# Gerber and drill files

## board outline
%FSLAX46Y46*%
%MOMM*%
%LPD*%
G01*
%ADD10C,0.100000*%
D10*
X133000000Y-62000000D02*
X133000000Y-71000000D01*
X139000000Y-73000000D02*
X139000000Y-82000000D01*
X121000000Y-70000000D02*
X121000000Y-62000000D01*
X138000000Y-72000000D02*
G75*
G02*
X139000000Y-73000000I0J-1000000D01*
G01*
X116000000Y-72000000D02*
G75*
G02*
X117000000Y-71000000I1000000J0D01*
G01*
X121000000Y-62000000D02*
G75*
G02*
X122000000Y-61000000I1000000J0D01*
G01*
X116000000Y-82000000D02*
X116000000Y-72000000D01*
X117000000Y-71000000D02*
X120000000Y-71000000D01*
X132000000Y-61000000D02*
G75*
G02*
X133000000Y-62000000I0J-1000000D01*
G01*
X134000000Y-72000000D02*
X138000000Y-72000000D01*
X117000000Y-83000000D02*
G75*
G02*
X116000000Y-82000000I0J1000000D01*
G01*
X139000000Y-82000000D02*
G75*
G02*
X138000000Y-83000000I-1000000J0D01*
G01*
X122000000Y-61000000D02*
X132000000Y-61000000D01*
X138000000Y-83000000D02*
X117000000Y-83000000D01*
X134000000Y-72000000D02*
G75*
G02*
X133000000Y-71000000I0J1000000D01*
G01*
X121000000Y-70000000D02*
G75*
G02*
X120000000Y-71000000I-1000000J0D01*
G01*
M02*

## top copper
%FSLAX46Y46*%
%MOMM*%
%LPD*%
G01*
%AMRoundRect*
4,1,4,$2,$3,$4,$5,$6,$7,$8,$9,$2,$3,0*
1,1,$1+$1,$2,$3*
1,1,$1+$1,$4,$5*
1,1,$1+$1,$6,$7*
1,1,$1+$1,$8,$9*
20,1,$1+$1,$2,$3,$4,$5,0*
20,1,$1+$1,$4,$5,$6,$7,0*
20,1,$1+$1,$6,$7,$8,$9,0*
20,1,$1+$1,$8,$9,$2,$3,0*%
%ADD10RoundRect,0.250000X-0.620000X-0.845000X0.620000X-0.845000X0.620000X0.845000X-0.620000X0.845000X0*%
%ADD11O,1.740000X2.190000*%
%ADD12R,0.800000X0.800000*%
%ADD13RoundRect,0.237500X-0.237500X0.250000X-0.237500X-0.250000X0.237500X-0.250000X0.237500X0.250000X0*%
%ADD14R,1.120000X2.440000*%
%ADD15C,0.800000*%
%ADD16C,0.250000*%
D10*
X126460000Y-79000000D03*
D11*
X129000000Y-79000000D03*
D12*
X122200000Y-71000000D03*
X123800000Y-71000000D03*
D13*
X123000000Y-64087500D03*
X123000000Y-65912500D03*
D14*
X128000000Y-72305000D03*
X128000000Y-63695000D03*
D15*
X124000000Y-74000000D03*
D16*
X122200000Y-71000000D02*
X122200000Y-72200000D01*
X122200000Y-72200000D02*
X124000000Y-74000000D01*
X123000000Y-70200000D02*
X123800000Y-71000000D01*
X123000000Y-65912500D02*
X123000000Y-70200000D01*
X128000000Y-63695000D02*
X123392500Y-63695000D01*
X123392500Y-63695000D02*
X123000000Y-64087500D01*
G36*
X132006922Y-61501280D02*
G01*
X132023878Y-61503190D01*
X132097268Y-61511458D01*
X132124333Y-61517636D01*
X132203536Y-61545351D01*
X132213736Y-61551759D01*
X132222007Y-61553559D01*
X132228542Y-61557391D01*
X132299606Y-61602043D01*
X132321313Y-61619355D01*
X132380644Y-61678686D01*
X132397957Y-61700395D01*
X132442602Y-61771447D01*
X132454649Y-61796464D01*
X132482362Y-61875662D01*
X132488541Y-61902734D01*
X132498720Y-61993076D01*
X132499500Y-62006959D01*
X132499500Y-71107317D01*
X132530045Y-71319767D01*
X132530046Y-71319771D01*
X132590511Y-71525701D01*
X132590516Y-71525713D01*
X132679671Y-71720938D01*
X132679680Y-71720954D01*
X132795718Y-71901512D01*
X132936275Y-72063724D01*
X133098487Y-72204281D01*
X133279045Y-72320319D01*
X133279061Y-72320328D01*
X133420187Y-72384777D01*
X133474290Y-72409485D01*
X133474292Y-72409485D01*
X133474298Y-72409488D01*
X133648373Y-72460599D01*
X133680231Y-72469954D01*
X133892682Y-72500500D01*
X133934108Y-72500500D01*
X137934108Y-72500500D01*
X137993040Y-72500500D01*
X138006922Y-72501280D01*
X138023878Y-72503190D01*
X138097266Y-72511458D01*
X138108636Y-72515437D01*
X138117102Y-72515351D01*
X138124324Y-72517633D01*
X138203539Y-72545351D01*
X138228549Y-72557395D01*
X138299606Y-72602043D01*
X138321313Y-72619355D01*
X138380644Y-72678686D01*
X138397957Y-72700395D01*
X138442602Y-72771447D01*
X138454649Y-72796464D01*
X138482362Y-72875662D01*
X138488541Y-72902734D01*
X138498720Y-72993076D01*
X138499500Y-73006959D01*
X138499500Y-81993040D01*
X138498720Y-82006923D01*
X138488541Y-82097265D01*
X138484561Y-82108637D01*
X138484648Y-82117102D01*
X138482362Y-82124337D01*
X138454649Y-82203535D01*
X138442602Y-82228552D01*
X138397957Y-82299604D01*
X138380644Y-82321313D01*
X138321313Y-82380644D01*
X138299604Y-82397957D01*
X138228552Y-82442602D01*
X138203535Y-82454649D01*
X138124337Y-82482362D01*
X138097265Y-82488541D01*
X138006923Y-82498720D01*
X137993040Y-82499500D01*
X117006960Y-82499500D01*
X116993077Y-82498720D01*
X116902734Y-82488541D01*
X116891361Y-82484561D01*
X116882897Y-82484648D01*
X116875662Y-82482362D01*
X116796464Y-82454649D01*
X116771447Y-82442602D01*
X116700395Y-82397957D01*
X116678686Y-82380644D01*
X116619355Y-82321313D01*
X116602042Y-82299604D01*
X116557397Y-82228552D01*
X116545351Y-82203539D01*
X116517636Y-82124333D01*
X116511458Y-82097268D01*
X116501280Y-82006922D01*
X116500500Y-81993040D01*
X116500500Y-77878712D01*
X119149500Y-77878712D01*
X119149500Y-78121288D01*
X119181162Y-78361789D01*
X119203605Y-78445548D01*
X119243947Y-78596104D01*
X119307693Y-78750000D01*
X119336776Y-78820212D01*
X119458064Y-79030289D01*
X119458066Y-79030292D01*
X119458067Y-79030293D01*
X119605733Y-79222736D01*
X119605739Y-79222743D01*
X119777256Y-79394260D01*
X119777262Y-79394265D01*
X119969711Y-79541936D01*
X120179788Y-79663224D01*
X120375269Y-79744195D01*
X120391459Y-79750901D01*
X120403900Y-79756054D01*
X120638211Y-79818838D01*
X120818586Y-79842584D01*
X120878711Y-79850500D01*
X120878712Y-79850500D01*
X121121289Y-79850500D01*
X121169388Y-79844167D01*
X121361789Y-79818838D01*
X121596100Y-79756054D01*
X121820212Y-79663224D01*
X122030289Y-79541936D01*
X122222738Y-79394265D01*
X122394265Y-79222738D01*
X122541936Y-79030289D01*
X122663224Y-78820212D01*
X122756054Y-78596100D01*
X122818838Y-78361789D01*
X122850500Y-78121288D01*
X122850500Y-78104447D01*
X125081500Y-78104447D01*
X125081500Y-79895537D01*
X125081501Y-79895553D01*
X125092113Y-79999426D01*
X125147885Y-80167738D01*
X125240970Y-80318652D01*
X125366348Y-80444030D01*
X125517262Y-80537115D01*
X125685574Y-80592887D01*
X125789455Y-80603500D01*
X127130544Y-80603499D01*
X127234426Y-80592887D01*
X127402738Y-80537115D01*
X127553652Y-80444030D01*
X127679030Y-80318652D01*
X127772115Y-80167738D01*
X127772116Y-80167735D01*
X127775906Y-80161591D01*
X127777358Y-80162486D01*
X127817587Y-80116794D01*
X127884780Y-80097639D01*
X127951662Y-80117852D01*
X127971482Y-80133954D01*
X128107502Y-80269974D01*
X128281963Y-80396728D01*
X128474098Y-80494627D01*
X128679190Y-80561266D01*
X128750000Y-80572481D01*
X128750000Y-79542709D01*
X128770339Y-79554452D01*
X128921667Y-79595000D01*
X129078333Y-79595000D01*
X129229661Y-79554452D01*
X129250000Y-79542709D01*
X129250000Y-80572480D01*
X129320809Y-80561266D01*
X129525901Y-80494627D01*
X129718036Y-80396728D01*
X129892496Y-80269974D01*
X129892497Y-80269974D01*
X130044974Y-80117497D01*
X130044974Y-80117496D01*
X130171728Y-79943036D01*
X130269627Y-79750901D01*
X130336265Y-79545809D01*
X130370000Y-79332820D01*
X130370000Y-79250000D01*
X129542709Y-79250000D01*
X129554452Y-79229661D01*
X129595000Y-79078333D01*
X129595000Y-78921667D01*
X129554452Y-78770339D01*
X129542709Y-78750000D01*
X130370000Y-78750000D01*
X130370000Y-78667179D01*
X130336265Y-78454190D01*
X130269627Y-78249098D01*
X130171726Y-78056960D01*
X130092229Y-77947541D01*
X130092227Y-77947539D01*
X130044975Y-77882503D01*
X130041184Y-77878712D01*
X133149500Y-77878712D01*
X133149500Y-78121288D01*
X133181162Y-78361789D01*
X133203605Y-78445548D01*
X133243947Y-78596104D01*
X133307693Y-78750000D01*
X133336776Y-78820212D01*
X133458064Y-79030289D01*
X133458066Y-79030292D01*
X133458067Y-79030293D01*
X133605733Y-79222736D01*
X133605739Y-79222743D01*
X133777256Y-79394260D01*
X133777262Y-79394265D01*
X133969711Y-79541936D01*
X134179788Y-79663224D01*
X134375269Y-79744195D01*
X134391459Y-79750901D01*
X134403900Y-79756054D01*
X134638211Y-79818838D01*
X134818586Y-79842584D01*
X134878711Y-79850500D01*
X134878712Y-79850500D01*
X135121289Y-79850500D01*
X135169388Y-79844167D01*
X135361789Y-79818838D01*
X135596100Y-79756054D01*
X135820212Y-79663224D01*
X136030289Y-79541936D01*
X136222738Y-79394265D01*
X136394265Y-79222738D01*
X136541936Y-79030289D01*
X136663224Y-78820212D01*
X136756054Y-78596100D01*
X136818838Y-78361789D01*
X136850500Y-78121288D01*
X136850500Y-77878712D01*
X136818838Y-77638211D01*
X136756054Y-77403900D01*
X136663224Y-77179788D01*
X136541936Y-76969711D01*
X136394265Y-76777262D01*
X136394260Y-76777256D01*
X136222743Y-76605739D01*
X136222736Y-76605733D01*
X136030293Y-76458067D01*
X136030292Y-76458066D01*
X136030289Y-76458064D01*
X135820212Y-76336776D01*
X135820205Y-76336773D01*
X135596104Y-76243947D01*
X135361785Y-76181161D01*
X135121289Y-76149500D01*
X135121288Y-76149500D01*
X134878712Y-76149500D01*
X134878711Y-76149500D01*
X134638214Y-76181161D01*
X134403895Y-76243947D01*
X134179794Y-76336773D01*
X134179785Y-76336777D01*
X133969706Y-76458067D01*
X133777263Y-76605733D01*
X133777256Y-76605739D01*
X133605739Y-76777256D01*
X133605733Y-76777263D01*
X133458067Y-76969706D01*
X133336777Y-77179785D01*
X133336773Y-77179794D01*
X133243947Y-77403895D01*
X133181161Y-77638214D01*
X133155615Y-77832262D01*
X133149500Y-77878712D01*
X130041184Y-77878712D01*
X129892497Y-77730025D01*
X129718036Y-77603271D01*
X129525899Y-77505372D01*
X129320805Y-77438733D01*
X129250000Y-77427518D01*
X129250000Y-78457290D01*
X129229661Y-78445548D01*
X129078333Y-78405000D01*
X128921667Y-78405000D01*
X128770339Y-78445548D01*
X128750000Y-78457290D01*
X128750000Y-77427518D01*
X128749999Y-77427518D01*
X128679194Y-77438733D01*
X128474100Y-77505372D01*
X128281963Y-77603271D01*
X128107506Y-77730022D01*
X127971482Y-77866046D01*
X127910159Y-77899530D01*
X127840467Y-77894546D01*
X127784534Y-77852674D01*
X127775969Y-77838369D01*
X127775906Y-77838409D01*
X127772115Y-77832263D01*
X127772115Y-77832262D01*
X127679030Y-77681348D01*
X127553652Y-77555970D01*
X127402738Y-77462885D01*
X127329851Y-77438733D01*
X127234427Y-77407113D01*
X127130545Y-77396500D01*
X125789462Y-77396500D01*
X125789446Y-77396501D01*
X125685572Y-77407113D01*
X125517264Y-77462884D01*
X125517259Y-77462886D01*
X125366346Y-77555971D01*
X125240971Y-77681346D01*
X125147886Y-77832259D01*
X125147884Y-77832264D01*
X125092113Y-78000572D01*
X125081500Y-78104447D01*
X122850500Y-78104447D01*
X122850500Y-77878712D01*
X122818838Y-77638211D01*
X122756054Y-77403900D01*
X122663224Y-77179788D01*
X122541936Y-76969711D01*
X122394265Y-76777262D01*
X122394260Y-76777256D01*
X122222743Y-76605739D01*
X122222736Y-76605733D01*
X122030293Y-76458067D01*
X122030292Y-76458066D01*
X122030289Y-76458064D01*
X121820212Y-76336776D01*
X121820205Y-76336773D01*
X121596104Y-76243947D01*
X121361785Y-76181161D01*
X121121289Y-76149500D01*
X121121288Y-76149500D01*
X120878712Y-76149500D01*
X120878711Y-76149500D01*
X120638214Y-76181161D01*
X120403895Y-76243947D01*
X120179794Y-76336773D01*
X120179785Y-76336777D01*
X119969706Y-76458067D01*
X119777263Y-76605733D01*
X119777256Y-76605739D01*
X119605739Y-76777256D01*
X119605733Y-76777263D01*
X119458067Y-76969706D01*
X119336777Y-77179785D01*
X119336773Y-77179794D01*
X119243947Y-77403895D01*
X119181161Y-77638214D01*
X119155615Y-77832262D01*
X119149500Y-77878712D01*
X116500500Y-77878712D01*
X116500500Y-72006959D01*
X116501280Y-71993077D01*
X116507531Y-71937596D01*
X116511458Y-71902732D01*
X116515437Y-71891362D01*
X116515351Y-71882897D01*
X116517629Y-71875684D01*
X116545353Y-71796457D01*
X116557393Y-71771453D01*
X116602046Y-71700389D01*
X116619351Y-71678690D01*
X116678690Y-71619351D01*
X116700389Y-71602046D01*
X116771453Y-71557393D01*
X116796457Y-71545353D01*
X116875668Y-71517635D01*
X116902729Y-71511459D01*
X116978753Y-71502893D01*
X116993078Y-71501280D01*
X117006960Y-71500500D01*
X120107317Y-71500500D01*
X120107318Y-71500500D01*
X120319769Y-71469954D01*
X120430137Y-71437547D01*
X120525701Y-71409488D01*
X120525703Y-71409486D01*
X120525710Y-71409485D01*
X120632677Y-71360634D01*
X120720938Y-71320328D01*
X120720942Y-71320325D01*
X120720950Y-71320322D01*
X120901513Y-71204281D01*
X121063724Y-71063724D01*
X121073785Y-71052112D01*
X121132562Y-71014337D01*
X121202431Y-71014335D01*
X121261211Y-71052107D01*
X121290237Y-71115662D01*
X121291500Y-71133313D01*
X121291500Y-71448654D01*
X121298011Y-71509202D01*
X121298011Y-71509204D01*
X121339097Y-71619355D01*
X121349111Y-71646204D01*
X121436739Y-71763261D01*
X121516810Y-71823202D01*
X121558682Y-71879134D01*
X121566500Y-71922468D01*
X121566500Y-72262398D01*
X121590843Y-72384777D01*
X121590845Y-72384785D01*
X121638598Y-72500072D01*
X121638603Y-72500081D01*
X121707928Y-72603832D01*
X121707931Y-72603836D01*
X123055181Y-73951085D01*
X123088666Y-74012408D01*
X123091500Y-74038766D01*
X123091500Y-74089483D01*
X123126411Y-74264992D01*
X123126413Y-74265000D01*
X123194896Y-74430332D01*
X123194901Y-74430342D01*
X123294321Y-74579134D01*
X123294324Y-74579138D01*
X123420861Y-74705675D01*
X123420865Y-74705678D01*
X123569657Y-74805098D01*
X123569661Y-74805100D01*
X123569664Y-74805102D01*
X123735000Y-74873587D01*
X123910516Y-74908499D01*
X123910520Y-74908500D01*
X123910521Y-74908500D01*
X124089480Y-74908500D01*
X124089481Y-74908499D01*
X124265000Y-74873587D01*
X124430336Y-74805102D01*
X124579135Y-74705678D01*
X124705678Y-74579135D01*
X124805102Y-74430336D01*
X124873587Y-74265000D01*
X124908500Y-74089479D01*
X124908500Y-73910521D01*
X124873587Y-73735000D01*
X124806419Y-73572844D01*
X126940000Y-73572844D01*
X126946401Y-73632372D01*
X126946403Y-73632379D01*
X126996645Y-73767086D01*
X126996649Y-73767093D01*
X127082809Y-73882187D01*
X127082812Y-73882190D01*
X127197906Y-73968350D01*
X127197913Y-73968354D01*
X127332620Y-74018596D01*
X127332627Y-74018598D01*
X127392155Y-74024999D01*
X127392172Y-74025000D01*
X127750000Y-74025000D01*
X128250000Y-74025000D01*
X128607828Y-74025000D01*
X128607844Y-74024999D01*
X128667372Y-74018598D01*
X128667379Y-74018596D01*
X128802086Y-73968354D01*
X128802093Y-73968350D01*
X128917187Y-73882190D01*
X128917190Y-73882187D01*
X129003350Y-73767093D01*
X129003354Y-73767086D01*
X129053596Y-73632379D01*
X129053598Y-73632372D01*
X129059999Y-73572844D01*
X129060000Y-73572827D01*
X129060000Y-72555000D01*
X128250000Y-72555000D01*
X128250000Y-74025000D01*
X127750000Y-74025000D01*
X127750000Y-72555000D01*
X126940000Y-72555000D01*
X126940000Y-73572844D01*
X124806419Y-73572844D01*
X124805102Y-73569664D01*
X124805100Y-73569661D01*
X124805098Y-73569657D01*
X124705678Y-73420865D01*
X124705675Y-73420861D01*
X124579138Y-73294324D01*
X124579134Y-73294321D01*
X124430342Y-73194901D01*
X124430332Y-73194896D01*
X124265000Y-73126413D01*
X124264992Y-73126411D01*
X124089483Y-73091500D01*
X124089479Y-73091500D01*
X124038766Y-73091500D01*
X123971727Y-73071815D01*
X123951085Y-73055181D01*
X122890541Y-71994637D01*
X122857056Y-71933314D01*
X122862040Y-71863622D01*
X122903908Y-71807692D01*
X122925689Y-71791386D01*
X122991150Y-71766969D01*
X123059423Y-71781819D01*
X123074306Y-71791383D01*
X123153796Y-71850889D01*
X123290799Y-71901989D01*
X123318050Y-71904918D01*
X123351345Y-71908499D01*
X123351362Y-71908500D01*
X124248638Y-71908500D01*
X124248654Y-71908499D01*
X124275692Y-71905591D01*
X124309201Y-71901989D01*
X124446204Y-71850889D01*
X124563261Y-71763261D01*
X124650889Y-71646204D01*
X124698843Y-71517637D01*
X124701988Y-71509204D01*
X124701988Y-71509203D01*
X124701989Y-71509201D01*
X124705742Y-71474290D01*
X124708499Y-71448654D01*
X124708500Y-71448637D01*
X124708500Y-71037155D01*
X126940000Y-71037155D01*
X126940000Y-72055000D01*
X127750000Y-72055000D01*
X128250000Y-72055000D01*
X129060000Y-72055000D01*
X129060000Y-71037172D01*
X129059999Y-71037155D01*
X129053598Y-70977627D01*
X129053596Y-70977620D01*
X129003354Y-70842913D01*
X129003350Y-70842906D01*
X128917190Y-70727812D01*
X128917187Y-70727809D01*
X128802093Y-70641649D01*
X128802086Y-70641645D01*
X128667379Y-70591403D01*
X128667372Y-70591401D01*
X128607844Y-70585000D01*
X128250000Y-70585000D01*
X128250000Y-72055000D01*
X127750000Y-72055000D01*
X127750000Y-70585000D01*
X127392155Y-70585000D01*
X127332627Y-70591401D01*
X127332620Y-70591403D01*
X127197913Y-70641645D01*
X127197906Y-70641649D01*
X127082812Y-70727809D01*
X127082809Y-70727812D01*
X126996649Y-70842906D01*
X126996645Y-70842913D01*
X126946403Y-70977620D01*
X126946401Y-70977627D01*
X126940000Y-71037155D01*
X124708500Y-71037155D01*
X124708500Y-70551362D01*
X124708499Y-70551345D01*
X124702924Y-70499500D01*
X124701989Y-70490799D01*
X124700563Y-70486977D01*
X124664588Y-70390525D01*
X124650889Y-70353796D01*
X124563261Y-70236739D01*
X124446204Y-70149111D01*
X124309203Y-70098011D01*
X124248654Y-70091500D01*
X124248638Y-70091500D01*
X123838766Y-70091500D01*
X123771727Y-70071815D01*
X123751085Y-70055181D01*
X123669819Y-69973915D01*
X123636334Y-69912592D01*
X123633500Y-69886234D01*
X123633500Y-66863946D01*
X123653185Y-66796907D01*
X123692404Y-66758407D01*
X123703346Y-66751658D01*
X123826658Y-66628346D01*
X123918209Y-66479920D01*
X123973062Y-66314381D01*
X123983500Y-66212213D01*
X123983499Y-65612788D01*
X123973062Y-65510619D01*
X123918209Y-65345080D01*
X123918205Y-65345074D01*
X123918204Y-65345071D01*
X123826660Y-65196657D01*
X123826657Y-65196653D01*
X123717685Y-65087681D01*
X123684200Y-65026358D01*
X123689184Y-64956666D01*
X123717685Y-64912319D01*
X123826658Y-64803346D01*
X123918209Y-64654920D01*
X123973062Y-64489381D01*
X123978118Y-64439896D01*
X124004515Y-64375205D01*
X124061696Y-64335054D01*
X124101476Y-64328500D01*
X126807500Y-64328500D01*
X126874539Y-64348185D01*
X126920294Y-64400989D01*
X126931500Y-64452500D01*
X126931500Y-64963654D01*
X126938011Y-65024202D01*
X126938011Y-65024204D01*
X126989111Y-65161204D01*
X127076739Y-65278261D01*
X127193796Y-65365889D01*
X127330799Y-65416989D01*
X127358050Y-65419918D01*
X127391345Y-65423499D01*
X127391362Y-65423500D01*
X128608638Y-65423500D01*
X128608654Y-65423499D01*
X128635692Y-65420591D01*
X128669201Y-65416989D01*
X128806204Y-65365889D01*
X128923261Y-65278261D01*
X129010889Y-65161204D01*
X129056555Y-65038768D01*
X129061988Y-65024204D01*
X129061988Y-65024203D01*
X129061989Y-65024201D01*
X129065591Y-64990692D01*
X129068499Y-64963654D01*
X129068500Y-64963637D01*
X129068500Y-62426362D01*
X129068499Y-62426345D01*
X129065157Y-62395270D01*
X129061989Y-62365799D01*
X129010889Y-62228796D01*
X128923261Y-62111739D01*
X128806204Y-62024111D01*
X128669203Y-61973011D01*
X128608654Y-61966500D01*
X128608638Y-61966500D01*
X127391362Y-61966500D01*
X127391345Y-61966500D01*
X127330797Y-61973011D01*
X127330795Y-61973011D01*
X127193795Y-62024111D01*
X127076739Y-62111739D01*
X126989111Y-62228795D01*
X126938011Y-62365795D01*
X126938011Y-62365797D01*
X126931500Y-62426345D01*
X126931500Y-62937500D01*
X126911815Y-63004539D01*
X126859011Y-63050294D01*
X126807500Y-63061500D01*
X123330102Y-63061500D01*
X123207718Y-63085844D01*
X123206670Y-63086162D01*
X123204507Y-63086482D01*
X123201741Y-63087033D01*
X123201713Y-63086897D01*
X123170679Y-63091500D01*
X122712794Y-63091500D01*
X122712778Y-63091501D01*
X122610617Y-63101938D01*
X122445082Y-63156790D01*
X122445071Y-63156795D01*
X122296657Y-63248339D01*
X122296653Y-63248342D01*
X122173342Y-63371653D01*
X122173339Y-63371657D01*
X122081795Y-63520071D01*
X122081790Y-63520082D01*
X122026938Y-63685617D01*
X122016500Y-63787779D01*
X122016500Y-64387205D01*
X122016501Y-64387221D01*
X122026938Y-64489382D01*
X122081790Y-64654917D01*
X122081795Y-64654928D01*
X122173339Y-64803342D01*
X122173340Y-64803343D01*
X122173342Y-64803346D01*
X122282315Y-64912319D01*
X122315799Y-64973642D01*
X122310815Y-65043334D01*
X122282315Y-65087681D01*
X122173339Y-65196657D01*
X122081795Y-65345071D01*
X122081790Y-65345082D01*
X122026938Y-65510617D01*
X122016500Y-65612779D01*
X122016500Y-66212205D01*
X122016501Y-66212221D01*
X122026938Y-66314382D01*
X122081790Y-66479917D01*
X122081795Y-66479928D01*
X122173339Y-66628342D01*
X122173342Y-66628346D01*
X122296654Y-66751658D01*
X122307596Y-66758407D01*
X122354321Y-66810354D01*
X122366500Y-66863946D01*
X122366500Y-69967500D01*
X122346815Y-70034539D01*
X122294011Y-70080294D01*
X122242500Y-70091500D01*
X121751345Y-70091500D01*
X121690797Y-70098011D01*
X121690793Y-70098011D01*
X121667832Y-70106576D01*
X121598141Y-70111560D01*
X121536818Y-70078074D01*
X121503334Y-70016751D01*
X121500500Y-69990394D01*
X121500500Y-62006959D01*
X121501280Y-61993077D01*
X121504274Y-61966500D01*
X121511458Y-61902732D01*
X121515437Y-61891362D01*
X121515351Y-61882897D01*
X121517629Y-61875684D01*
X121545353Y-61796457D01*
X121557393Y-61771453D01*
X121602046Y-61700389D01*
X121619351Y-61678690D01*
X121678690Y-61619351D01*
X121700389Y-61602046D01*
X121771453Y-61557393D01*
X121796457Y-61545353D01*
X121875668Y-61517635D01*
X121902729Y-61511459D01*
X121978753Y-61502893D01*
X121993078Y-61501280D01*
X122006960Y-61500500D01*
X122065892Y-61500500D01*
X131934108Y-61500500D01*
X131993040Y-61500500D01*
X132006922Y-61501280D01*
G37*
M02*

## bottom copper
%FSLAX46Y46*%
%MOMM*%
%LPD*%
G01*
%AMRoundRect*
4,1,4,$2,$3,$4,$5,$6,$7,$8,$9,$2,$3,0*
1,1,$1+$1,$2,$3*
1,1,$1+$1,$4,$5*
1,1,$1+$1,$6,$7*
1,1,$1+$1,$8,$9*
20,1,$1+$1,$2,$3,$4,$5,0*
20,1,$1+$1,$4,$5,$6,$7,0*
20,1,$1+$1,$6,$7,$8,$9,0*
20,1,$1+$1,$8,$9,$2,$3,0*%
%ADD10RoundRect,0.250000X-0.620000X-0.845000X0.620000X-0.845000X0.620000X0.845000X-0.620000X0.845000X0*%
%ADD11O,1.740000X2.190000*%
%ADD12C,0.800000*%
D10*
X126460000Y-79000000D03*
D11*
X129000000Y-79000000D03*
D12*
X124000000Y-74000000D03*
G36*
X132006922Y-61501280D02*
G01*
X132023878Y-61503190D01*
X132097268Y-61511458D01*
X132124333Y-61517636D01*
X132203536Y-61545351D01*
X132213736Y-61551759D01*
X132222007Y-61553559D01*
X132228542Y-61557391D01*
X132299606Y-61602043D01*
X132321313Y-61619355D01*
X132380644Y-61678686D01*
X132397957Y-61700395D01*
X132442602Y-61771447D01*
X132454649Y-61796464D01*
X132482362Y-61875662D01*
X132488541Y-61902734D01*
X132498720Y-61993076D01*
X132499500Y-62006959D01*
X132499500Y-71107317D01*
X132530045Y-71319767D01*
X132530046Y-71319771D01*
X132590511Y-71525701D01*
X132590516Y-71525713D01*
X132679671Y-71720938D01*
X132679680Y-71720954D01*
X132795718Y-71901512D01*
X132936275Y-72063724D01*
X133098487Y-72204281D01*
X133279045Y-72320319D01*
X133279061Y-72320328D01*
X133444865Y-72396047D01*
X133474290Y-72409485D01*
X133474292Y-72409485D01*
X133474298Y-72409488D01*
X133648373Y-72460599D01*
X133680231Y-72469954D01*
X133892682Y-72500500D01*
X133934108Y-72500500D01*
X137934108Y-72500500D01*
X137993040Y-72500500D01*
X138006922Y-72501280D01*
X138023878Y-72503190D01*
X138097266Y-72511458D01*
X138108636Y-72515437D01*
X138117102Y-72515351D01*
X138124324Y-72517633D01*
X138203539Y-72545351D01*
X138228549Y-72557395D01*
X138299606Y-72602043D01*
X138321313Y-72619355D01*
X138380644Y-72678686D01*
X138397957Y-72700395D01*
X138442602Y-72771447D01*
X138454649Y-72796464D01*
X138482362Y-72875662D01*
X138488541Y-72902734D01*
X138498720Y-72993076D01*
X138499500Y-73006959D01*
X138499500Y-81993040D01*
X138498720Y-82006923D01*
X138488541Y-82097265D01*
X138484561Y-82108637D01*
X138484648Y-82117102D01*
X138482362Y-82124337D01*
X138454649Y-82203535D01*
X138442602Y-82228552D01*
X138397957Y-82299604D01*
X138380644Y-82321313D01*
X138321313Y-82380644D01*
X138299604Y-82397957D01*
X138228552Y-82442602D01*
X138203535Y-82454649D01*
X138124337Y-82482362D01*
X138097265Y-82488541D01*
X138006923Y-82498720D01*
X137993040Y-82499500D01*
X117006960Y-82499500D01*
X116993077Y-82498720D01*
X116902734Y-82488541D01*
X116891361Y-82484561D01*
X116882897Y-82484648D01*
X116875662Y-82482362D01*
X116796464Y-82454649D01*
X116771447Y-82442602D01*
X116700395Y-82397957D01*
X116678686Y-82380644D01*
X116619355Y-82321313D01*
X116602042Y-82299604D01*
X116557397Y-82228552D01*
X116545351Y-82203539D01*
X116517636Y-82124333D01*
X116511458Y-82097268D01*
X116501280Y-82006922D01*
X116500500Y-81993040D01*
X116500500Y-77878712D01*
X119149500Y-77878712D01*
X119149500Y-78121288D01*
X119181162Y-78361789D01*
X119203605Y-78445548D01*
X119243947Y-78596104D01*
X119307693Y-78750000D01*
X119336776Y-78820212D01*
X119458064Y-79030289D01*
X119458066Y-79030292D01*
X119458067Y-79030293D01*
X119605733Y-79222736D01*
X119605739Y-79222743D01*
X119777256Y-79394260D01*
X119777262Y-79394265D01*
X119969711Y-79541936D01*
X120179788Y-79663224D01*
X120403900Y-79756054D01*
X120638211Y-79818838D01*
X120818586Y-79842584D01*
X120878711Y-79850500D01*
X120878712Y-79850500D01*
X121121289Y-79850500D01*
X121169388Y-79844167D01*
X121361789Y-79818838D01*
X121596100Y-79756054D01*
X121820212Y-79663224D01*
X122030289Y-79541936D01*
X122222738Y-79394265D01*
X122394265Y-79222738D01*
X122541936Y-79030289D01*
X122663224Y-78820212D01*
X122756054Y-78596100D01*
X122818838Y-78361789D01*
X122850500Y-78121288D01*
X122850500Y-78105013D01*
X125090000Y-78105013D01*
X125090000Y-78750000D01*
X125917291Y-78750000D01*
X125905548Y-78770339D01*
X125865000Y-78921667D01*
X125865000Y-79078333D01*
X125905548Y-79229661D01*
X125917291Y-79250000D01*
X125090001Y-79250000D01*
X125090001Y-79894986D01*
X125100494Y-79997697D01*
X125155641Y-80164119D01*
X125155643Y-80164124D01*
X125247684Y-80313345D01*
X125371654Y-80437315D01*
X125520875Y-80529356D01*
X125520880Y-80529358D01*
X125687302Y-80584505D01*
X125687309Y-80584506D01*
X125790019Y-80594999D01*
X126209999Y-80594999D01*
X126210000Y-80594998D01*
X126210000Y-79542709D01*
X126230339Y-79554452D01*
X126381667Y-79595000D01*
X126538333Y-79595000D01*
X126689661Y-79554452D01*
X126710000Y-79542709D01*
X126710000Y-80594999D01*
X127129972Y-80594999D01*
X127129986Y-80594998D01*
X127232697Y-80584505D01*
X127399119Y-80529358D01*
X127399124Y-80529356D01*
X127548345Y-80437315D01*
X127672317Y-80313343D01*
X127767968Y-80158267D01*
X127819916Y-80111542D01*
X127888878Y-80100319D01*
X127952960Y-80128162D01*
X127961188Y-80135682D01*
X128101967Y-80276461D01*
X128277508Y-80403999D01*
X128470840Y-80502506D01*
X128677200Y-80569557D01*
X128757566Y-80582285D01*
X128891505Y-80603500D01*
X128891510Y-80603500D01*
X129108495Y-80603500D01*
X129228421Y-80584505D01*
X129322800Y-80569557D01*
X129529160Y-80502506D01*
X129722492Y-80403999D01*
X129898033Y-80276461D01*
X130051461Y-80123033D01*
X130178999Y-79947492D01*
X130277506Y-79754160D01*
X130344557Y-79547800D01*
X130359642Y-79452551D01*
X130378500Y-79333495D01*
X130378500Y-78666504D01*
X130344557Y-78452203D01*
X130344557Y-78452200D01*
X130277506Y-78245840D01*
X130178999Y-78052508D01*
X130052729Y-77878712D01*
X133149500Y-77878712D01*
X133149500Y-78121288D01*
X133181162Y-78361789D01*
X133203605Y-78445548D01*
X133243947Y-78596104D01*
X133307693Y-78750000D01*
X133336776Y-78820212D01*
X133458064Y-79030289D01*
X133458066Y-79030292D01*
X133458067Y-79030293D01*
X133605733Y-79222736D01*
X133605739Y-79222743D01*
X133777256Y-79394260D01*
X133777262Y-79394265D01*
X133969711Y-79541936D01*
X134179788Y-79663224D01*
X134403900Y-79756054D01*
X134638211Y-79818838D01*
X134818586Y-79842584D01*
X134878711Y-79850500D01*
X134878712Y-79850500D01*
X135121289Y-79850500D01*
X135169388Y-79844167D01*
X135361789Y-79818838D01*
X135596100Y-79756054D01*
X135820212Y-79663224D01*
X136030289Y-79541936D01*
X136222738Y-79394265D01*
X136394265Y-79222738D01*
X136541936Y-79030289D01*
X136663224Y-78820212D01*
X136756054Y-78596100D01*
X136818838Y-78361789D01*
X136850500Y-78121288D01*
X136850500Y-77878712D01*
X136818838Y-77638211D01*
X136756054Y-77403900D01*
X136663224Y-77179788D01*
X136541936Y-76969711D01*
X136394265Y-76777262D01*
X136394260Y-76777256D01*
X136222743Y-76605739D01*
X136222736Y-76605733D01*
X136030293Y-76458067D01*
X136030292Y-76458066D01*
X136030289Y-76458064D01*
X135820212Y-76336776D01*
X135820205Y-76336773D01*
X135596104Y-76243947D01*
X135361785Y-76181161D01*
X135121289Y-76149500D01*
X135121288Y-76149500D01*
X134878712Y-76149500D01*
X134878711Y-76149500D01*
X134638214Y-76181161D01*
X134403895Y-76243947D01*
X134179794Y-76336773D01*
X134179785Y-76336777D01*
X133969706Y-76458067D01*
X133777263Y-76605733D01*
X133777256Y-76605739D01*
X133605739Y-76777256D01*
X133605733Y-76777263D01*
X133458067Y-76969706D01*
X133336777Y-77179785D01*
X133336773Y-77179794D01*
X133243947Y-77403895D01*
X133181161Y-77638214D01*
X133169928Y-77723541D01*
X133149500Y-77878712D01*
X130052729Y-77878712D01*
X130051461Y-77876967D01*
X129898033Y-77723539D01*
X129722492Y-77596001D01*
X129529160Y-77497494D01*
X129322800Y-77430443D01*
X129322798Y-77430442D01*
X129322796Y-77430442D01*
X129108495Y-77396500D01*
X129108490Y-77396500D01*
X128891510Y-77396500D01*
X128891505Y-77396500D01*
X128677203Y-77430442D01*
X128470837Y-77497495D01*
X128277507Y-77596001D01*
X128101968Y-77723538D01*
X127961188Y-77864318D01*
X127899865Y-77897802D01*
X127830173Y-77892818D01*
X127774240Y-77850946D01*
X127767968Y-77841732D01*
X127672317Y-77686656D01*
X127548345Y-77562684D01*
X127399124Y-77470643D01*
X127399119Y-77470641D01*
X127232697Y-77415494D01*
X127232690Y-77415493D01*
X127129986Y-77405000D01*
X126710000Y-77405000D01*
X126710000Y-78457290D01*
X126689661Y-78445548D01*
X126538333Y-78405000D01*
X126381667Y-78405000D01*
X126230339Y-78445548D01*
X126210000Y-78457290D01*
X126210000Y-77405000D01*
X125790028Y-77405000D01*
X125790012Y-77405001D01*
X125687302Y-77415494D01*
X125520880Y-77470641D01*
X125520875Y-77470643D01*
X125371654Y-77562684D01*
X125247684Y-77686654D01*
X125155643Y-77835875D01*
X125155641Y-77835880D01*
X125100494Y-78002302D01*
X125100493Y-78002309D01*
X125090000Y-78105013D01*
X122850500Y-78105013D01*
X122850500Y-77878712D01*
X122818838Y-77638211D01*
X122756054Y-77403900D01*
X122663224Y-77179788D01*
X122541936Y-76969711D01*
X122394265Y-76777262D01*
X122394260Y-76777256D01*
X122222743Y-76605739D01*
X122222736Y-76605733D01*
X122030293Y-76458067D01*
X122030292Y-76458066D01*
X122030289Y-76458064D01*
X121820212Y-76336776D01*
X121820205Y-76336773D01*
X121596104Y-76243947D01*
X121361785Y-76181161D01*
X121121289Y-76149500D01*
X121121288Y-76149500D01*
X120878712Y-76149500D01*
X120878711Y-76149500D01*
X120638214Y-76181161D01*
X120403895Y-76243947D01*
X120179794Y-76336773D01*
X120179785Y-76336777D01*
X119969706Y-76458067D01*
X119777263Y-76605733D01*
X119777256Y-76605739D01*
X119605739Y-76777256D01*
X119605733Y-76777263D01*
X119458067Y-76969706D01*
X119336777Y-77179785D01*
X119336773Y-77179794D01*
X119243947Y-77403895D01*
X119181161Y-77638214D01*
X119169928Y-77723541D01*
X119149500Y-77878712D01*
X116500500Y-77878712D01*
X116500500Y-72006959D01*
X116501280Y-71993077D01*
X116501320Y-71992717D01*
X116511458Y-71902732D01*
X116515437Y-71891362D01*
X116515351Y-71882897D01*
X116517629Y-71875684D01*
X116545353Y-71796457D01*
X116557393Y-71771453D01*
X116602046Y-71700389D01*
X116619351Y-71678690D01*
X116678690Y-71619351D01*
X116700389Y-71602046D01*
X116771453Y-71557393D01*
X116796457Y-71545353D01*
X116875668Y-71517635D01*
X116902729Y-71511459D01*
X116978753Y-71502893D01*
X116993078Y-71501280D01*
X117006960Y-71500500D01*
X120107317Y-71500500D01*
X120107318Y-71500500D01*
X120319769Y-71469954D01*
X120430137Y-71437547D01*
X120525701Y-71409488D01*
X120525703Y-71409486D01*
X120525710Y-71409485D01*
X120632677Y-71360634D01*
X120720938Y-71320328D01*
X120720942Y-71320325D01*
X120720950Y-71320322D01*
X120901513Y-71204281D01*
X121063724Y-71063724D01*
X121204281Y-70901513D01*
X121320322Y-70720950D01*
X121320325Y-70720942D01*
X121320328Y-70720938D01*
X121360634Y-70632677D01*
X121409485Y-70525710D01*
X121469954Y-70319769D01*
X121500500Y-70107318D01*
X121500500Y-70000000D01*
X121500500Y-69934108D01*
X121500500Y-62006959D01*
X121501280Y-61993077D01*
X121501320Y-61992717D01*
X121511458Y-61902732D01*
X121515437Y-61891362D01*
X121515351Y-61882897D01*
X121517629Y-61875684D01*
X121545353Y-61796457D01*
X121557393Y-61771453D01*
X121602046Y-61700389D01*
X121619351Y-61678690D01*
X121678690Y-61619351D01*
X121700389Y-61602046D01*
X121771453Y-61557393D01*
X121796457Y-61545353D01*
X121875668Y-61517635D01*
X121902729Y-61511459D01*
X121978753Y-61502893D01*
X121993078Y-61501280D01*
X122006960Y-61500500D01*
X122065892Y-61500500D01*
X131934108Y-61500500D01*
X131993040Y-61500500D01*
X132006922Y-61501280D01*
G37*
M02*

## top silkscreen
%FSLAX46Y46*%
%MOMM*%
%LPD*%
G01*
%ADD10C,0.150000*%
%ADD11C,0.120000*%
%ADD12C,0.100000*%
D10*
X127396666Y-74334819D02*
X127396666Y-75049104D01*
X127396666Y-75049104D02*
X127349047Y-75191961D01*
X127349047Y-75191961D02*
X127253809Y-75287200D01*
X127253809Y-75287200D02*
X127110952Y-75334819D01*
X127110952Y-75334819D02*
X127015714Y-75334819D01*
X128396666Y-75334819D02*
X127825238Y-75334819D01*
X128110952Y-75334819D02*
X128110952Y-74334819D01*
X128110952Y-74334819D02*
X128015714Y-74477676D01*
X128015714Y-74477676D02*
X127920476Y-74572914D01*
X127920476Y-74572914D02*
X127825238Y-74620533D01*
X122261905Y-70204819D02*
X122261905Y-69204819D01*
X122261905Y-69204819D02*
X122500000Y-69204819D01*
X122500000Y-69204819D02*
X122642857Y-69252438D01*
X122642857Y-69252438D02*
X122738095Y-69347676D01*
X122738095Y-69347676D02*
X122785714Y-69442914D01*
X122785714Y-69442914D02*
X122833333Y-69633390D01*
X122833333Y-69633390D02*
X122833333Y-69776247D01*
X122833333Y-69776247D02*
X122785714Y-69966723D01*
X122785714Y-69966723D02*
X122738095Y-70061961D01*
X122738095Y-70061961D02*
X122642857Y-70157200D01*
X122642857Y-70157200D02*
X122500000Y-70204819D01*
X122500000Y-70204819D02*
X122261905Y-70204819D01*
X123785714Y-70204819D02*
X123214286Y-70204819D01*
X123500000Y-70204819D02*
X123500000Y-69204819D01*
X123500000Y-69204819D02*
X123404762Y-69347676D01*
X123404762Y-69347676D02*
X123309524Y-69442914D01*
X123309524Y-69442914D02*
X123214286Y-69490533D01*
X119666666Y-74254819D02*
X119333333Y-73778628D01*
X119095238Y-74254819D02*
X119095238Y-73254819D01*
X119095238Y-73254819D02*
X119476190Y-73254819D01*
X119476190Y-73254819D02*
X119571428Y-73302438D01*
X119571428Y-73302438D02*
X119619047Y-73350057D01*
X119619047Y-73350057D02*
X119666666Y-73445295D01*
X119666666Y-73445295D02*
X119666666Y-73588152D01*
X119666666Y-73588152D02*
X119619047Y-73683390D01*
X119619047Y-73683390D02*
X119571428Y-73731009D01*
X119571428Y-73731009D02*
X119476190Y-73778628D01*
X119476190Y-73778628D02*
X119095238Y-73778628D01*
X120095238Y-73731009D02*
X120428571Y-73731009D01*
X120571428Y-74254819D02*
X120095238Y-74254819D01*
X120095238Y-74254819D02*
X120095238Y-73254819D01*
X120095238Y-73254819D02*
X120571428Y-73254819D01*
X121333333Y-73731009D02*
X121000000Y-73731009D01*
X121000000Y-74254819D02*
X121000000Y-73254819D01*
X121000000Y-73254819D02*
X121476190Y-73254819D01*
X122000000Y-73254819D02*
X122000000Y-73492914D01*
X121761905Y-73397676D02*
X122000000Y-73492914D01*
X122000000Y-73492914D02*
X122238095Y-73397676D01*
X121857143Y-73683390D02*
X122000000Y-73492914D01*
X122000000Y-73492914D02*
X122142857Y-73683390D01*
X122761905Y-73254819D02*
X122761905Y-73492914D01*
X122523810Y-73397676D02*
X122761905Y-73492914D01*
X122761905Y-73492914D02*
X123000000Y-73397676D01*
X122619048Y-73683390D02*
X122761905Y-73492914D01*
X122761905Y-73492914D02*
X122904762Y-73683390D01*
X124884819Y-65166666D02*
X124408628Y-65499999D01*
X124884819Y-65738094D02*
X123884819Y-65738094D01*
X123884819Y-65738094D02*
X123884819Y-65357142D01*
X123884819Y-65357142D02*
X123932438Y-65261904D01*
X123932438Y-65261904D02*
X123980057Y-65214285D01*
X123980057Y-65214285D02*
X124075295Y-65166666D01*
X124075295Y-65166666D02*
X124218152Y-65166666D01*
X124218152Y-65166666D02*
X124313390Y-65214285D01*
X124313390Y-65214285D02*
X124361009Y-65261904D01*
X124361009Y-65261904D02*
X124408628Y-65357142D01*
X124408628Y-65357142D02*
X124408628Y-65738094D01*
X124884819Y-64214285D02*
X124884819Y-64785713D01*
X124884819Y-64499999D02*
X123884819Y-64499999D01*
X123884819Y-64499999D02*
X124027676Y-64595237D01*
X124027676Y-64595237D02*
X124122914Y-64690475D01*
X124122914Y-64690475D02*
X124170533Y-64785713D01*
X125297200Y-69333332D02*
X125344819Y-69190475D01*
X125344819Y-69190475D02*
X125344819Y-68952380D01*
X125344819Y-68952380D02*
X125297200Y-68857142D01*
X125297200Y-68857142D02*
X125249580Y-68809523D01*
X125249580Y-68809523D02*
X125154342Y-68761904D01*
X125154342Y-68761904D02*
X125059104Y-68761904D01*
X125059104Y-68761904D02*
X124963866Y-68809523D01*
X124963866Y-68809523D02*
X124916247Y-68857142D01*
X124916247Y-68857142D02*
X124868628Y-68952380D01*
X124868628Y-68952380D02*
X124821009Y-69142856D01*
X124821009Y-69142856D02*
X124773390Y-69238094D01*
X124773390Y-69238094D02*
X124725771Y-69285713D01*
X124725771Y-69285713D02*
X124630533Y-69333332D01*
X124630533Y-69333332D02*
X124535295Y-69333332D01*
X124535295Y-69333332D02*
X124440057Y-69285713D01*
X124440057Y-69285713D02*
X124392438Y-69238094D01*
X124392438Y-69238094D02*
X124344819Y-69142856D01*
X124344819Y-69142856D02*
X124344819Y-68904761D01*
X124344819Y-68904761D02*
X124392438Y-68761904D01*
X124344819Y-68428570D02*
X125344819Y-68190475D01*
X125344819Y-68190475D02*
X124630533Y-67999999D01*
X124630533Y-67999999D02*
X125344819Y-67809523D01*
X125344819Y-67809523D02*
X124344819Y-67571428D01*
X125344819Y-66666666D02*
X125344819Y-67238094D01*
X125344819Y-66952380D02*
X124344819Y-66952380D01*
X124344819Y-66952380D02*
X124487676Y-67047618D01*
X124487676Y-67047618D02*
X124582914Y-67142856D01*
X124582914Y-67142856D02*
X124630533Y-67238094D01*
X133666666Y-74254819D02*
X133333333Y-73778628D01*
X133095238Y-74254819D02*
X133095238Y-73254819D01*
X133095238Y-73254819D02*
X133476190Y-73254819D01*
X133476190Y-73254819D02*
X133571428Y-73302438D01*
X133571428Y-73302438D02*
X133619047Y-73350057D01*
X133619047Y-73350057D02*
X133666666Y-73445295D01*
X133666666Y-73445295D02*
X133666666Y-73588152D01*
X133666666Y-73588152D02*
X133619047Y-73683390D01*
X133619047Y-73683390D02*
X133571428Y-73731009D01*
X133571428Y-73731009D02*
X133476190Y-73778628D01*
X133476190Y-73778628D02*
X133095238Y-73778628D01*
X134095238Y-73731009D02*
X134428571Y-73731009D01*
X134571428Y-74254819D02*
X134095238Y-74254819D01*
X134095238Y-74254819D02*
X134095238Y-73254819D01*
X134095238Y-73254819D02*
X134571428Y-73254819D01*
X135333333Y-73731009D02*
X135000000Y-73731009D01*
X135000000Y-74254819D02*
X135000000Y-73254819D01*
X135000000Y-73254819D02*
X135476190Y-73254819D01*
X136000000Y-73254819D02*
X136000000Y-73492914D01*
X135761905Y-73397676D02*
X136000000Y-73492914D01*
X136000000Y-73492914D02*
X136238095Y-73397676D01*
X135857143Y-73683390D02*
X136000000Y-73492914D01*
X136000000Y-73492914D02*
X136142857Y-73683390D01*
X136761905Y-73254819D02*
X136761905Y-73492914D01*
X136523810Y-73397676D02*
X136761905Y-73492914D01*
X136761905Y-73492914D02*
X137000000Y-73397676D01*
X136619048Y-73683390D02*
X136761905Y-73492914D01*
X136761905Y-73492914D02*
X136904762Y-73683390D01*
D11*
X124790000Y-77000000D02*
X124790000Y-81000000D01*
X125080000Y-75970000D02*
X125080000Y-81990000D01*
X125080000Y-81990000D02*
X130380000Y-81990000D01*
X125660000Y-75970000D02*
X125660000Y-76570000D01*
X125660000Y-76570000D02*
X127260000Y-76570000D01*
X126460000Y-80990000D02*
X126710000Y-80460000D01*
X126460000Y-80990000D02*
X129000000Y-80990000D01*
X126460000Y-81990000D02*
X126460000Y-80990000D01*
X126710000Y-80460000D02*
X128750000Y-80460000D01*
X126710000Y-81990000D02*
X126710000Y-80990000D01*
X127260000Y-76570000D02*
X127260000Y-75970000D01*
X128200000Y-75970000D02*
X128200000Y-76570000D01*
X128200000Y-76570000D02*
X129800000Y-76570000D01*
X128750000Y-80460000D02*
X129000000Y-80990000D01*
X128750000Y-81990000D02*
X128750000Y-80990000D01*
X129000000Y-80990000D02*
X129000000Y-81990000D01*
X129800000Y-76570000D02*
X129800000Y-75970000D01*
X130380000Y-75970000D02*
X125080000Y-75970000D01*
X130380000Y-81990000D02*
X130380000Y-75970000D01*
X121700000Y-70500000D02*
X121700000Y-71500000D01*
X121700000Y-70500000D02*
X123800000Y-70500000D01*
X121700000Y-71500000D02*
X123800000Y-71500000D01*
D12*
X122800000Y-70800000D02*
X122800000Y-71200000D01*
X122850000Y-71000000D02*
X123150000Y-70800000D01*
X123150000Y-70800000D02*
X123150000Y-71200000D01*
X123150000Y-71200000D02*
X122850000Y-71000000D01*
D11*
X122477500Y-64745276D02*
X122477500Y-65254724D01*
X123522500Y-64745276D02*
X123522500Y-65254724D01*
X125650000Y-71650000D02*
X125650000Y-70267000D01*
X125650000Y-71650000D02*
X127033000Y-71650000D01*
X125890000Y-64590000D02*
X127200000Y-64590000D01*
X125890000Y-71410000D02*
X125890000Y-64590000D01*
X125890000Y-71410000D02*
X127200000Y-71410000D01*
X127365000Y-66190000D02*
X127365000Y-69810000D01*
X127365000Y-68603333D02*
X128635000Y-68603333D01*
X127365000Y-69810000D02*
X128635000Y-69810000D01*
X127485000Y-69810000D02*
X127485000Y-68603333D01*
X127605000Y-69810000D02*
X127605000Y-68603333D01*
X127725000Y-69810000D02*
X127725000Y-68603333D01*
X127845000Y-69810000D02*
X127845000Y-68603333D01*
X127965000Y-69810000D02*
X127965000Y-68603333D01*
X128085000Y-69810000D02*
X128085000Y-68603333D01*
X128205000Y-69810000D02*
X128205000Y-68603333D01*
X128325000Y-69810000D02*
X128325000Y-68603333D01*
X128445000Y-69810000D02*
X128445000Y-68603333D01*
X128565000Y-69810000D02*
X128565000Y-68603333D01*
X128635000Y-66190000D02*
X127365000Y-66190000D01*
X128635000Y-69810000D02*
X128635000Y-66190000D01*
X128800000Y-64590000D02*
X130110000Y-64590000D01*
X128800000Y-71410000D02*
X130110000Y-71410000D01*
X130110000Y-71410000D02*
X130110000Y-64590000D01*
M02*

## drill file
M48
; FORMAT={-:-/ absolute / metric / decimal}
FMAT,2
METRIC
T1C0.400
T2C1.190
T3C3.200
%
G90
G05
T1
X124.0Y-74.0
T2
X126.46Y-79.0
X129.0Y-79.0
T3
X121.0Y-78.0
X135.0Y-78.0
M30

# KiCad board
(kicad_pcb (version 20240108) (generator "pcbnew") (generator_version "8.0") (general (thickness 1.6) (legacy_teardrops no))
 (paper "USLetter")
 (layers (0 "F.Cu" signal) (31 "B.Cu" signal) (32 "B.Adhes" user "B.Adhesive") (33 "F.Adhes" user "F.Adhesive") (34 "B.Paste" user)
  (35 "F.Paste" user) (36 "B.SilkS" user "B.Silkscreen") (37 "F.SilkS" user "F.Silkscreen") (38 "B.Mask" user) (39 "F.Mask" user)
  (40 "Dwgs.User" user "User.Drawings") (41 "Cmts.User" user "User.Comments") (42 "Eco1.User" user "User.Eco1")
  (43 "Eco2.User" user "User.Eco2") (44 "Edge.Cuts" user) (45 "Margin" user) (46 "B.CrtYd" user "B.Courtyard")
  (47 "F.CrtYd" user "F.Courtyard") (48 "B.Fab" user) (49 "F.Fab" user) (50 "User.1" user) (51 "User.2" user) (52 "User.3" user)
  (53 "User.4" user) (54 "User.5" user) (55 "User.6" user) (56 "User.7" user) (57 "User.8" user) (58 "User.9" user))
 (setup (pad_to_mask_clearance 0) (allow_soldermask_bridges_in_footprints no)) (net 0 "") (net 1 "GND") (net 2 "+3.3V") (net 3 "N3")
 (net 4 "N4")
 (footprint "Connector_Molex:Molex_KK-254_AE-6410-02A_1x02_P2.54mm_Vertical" (layer "F.Cu") (at 126.46 79)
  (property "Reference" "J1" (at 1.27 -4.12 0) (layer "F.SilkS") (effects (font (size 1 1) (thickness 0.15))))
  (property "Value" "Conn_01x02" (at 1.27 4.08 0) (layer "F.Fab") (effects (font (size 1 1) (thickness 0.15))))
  (fp_line (start -1.67 -2) (end -1.67 2) (stroke (width 0.12) (type solid)) (layer "F.SilkS"))
  (fp_line (start -1.38 -3.03) (end -1.38 2.99) (stroke (width 0.12) (type solid)) (layer "F.SilkS"))
  (fp_line (start -1.38 2.99) (end 3.92 2.99) (stroke (width 0.12) (type solid)) (layer "F.SilkS"))
  (fp_line (start -0.8 -3.03) (end -0.8 -2.43) (stroke (width 0.12) (type solid)) (layer "F.SilkS"))
  (fp_line (start -0.8 -2.43) (end 0.8 -2.43) (stroke (width 0.12) (type solid)) (layer "F.SilkS"))
  (fp_line (start 0 1.99) (end 0.25 1.46) (stroke (width 0.12) (type solid)) (layer "F.SilkS"))
  (fp_line (start 0 1.99) (end 2.54 1.99) (stroke (width 0.12) (type solid)) (layer "F.SilkS"))
  (fp_line (start 0 2.99) (end 0 1.99) (stroke (width 0.12) (type solid)) (layer "F.SilkS"))
  (fp_line (start 0.25 1.46) (end 2.29 1.46) (stroke (width 0.12) (type solid)) (layer "F.SilkS"))
  (fp_line (start 0.25 2.99) (end 0.25 1.99) (stroke (width 0.12) (type solid)) (layer "F.SilkS"))
  (fp_line (start 0.8 -2.43) (end 0.8 -3.03) (stroke (width 0.12) (type solid)) (layer "F.SilkS"))
  (fp_line (start 1.74 -3.03) (end 1.74 -2.43) (stroke (width 0.12) (type solid)) (layer "F.SilkS"))
  (fp_line (start 1.74 -2.43) (end 3.34 -2.43) (stroke (width 0.12) (type solid)) (layer "F.SilkS"))
  (fp_line (start 2.29 1.46) (end 2.54 1.99) (stroke (width 0.12) (type solid)) (layer "F.SilkS"))
  (fp_line (start 2.29 2.99) (end 2.29 1.99) (stroke (width 0.12) (type solid)) (layer "F.SilkS"))
  (fp_line (start 2.54 1.99) (end 2.54 2.99) (stroke (width 0.12) (type solid)) (layer "F.SilkS"))
  (fp_line (start 3.34 -2.43) (end 3.34 -3.03) (stroke (width 0.12) (type solid)) (layer "F.SilkS"))
  (fp_line (start 3.92 -3.03) (end -1.38 -3.03) (stroke (width 0.12) (type solid)) (layer "F.SilkS"))
  (fp_line (start 3.92 2.99) (end 3.92 -3.03) (stroke (width 0.12) (type solid)) (layer "F.SilkS"))
  (pad "1" thru_hole roundrect (at 0 0) (size 1.74 2.19) (drill 1.19) (layers "*.Cu" "*.Mask") (remove_unused_layers no)
   (roundrect_rratio 0.143678) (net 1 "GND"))
  (pad "2" thru_hole oval (at 2.54 0) (size 1.74 2.19) (drill 1.19) (layers "*.Cu" "*.Mask") (remove_unused_layers no) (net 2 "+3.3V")))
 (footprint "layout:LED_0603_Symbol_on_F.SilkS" (layer "F.Cu") (at 123 71)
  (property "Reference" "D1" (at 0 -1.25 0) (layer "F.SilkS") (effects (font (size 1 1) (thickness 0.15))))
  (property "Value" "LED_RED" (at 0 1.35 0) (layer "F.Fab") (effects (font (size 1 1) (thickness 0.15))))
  (fp_line (start -1.3 -0.5) (end -1.3 0.5) (stroke (width 0.12) (type solid)) (layer "F.SilkS"))
  (fp_line (start -1.3 -0.5) (end 0.8 -0.5) (stroke (width 0.12) (type solid)) (layer "F.SilkS"))
  (fp_line (start -1.3 0.5) (end 0.8 0.5) (stroke (width 0.12) (type solid)) (layer "F.SilkS"))
  (fp_line (start -0.2 -0.2) (end -0.2 0.2) (stroke (width 0.1) (type solid)) (layer "F.SilkS"))
  (fp_line (start -0.15 0) (end 0.15 -0.2) (stroke (width 0.1) (type solid)) (layer "F.SilkS"))
  (fp_line (start 0.15 -0.2) (end 0.15 0.2) (stroke (width 0.1) (type solid)) (layer "F.SilkS"))
  (fp_line (start 0.15 0.2) (end -0.15 0) (stroke (width 0.1) (type solid)) (layer "F.SilkS"))
  (pad "1" smd rect (at -0.8 0 180) (size 0.8 0.8) (layers "F.Cu" "F.Paste" "F.Mask") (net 1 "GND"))
  (pad "2" smd rect (at 0.8 0 180) (size 0.8 0.8) (layers "F.Cu" "F.Paste" "F.Mask") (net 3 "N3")))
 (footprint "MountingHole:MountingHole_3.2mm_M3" (layer "F.Cu") (at 121 78)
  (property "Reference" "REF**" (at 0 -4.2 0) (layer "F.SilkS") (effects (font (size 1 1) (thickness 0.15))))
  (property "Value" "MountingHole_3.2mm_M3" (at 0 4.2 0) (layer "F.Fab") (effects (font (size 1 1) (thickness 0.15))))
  (pad "" np_thru_hole circle (at 0 0) (size 3.2 3.2) (drill 3.2) (layers "*.Cu" "*.Mask")))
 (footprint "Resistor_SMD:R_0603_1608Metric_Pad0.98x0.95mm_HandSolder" (layer "F.Cu") (at 123 65 -90)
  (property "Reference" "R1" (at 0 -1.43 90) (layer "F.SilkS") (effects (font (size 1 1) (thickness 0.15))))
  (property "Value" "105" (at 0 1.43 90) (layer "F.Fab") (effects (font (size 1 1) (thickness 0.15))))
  (fp_line (start -0.254724 0.5225) (end 0.254724 0.5225) (stroke (width 0.12) (type solid)) (layer "F.SilkS"))
  (fp_line (start -0.254724 -0.5225) (end 0.254724 -0.5225) (stroke (width 0.12) (type solid)) (layer "F.SilkS"))
  (pad "1" smd roundrect (at -0.9125 0 270) (size 0.975 0.95) (layers "F.Cu" "F.Paste" "F.Mask") (roundrect_rratio 0.25) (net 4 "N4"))
  (pad "2" smd roundrect (at 0.9125 0 270) (size 0.975 0.95) (layers "F.Cu" "F.Paste" "F.Mask") (roundrect_rratio 0.25) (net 3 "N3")))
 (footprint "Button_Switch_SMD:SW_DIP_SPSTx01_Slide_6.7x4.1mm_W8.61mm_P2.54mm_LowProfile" (layer "F.Cu") (at 128 68 90)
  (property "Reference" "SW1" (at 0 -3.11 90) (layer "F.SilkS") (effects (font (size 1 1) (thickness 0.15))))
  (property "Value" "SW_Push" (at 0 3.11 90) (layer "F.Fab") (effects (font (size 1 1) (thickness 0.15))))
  (fp_line (start -3.65 -2.35) (end -2.267 -2.35) (stroke (width 0.12) (type solid)) (layer "F.SilkS"))
  (fp_line (start -3.65 -2.35) (end -3.65 -0.967) (stroke (width 0.12) (type solid)) (layer "F.SilkS"))
  (fp_line (start 3.41 -2.11) (end 3.41 -0.8) (stroke (width 0.12) (type solid)) (layer "F.SilkS"))
  (fp_line (start -3.41 -2.11) (end 3.41 -2.11) (stroke (width 0.12) (type solid)) (layer "F.SilkS"))
  (fp_line (start -3.41 -2.11) (end -3.41 -0.8) (stroke (width 0.12) (type solid)) (layer "F.SilkS"))
  (fp_line (start 1.81 -0.635) (end -1.81 -0.635) (stroke (width 0.12) (type solid)) (layer "F.SilkS"))
  (fp_line (start -0.603333 -0.635) (end -0.603333 0.635) (stroke (width 0.12) (type solid)) (layer "F.SilkS"))
  (fp_line (start -1.81 -0.635) (end -1.81 0.635) (stroke (width 0.12) (type solid)) (layer "F.SilkS"))
  (fp_line (start -1.81 -0.515) (end -0.603333 -0.515) (stroke (width 0.12) (type solid)) (layer "F.SilkS"))
  (fp_line (start -1.81 -0.395) (end -0.603333 -0.395) (stroke (width 0.12) (type solid)) (layer "F.SilkS"))
  (fp_line (start -1.81 -0.275) (end -0.603333 -0.275) (stroke (width 0.12) (type solid)) (layer "F.SilkS"))
  (fp_line (start -1.81 -0.155) (end -0.603333 -0.155) (stroke (width 0.12) (type solid)) (layer "F.SilkS"))
  (fp_line (start -1.81 -0.035) (end -0.603333 -0.035) (stroke (width 0.12) (type solid)) (layer "F.SilkS"))
  (fp_line (start -1.81 0.085) (end -0.603333 0.085) (stroke (width 0.12) (type solid)) (layer "F.SilkS"))
  (fp_line (start -1.81 0.205) (end -0.603333 0.205) (stroke (width 0.12) (type solid)) (layer "F.SilkS"))
  (fp_line (start -1.81 0.325) (end -0.603333 0.325) (stroke (width 0.12) (type solid)) (layer "F.SilkS"))
  (fp_line (start -1.81 0.445) (end -0.603333 0.445) (stroke (width 0.12) (type solid)) (layer "F.SilkS"))
  (fp_line (start -1.81 0.565) (end -0.603333 0.565) (stroke (width 0.12) (type solid)) (layer "F.SilkS"))
  (fp_line (start 1.81 0.635) (end 1.81 -0.635) (stroke (width 0.12) (type solid)) (layer "F.SilkS"))
  (fp_line (start -1.81 0.635) (end 1.81 0.635) (stroke (width 0.12) (type solid)) (layer "F.SilkS"))
  (fp_line (start 3.41 0.8) (end 3.41 2.11) (stroke (width 0.12) (type solid)) (layer "F.SilkS"))
  (fp_line (start -3.41 0.8) (end -3.41 2.11) (stroke (width 0.12) (type solid)) (layer "F.SilkS"))
  (fp_line (start -3.41 2.11) (end 3.41 2.11) (stroke (width 0.12) (type solid)) (layer "F.SilkS"))
  (pad "1" smd rect (at -4.305 0 90) (size 2.44 1.12) (layers "F.Cu" "F.Paste" "F.Mask") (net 2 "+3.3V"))
  (pad "2" smd rect (at 4.305 0 90) (size 2.44 1.12) (layers "F.Cu" "F.Paste" "F.Mask") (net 4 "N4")))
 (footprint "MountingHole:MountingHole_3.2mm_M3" (layer "F.Cu") (at 135 78)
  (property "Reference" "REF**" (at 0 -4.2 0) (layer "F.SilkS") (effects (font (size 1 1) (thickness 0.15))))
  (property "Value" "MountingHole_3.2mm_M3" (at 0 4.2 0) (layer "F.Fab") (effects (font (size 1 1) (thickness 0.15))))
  (pad "" np_thru_hole circle (at 0 0) (size 3.2 3.2) (drill 3.2) (layers "*.Cu" "*.Mask")))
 (gr_line (start 133 62) (end 133 71) (stroke (width 0.1) (type default)) (layer "Edge.Cuts"))
 (gr_line (start 139 73) (end 139 82) (stroke (width 0.1) (type default)) (layer "Edge.Cuts"))
 (gr_line (start 121 70) (end 121 62) (stroke (width 0.1) (type default)) (layer "Edge.Cuts"))
 (gr_arc (start 138 72) (mid 138.707107 72.292893) (end 139 73) (stroke (width 0.1) (type default)) (layer "Edge.Cuts"))
 (gr_arc (start 116 72) (mid 116.292893 71.292893) (end 117 71) (stroke (width 0.1) (type default)) (layer "Edge.Cuts"))
 (gr_arc (start 121 62) (mid 121.292893 61.292893) (end 122 61) (stroke (width 0.1) (type default)) (layer "Edge.Cuts"))
 (gr_line (start 116 82) (end 116 72) (stroke (width 0.1) (type default)) (layer "Edge.Cuts"))
 (gr_line (start 117 71) (end 120 71) (stroke (width 0.1) (type default)) (layer "Edge.Cuts"))
 (gr_arc (start 132 61) (mid 132.707107 61.292893) (end 133 62) (stroke (width 0.1) (type default)) (layer "Edge.Cuts"))
 (gr_line (start 134 72) (end 138 72) (stroke (width 0.1) (type default)) (layer "Edge.Cuts"))
 (gr_arc (start 117 83) (mid 116.292893 82.707107) (end 116 82) (stroke (width 0.1) (type default)) (layer "Edge.Cuts"))
 (gr_arc (start 139 82) (mid 138.707107 82.707107) (end 138 83) (stroke (width 0.1) (type default)) (layer "Edge.Cuts"))
 (gr_line (start 122 61) (end 132 61) (stroke (width 0.1) (type default)) (layer "Edge.Cuts"))
 (gr_line (start 138 83) (end 117 83) (stroke (width 0.1) (type default)) (layer "Edge.Cuts"))
 (gr_arc (start 134 72) (mid 133.292893 71.707107) (end 133 71) (stroke (width 0.1) (type default)) (layer "Edge.Cuts"))
 (gr_arc (start 121 70) (mid 120.707107 70.707107) (end 120 71) (stroke (width 0.1) (type default)) (layer "Edge.Cuts"))
 (segment (start 122.2 71) (end 122.2 72.2) (width 0.25) (layer "F.Cu") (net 1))
 (segment (start 122.2 72.2) (end 124 74) (width 0.25) (layer "F.Cu") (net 1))
 (via (at 124 74) (size 0.8) (drill 0.4) (layers "F.Cu" "B.Cu") (free yes) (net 1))
 (segment (start 123 70.2) (end 123.8 71) (width 0.25) (layer "F.Cu") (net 3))
 (segment (start 123 65.9125) (end 123 70.2) (width 0.25) (layer "F.Cu") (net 3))
 (segment (start 128 63.695) (end 123.3925 63.695) (width 0.25) (layer "F.Cu") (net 4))
 (segment (start 123.3925 63.695) (end 123 64.0875) (width 0.25) (layer "F.Cu") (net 4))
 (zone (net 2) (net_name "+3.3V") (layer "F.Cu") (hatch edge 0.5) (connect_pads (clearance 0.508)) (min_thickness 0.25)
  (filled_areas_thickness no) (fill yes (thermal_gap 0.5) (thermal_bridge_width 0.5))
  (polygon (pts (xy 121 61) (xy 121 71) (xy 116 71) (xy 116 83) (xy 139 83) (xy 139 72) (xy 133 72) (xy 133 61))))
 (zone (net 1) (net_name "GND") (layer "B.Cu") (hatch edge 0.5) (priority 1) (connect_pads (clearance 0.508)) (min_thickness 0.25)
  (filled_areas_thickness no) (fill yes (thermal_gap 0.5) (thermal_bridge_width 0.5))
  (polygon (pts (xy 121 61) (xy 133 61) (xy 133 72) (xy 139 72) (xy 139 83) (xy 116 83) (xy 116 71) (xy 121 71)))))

